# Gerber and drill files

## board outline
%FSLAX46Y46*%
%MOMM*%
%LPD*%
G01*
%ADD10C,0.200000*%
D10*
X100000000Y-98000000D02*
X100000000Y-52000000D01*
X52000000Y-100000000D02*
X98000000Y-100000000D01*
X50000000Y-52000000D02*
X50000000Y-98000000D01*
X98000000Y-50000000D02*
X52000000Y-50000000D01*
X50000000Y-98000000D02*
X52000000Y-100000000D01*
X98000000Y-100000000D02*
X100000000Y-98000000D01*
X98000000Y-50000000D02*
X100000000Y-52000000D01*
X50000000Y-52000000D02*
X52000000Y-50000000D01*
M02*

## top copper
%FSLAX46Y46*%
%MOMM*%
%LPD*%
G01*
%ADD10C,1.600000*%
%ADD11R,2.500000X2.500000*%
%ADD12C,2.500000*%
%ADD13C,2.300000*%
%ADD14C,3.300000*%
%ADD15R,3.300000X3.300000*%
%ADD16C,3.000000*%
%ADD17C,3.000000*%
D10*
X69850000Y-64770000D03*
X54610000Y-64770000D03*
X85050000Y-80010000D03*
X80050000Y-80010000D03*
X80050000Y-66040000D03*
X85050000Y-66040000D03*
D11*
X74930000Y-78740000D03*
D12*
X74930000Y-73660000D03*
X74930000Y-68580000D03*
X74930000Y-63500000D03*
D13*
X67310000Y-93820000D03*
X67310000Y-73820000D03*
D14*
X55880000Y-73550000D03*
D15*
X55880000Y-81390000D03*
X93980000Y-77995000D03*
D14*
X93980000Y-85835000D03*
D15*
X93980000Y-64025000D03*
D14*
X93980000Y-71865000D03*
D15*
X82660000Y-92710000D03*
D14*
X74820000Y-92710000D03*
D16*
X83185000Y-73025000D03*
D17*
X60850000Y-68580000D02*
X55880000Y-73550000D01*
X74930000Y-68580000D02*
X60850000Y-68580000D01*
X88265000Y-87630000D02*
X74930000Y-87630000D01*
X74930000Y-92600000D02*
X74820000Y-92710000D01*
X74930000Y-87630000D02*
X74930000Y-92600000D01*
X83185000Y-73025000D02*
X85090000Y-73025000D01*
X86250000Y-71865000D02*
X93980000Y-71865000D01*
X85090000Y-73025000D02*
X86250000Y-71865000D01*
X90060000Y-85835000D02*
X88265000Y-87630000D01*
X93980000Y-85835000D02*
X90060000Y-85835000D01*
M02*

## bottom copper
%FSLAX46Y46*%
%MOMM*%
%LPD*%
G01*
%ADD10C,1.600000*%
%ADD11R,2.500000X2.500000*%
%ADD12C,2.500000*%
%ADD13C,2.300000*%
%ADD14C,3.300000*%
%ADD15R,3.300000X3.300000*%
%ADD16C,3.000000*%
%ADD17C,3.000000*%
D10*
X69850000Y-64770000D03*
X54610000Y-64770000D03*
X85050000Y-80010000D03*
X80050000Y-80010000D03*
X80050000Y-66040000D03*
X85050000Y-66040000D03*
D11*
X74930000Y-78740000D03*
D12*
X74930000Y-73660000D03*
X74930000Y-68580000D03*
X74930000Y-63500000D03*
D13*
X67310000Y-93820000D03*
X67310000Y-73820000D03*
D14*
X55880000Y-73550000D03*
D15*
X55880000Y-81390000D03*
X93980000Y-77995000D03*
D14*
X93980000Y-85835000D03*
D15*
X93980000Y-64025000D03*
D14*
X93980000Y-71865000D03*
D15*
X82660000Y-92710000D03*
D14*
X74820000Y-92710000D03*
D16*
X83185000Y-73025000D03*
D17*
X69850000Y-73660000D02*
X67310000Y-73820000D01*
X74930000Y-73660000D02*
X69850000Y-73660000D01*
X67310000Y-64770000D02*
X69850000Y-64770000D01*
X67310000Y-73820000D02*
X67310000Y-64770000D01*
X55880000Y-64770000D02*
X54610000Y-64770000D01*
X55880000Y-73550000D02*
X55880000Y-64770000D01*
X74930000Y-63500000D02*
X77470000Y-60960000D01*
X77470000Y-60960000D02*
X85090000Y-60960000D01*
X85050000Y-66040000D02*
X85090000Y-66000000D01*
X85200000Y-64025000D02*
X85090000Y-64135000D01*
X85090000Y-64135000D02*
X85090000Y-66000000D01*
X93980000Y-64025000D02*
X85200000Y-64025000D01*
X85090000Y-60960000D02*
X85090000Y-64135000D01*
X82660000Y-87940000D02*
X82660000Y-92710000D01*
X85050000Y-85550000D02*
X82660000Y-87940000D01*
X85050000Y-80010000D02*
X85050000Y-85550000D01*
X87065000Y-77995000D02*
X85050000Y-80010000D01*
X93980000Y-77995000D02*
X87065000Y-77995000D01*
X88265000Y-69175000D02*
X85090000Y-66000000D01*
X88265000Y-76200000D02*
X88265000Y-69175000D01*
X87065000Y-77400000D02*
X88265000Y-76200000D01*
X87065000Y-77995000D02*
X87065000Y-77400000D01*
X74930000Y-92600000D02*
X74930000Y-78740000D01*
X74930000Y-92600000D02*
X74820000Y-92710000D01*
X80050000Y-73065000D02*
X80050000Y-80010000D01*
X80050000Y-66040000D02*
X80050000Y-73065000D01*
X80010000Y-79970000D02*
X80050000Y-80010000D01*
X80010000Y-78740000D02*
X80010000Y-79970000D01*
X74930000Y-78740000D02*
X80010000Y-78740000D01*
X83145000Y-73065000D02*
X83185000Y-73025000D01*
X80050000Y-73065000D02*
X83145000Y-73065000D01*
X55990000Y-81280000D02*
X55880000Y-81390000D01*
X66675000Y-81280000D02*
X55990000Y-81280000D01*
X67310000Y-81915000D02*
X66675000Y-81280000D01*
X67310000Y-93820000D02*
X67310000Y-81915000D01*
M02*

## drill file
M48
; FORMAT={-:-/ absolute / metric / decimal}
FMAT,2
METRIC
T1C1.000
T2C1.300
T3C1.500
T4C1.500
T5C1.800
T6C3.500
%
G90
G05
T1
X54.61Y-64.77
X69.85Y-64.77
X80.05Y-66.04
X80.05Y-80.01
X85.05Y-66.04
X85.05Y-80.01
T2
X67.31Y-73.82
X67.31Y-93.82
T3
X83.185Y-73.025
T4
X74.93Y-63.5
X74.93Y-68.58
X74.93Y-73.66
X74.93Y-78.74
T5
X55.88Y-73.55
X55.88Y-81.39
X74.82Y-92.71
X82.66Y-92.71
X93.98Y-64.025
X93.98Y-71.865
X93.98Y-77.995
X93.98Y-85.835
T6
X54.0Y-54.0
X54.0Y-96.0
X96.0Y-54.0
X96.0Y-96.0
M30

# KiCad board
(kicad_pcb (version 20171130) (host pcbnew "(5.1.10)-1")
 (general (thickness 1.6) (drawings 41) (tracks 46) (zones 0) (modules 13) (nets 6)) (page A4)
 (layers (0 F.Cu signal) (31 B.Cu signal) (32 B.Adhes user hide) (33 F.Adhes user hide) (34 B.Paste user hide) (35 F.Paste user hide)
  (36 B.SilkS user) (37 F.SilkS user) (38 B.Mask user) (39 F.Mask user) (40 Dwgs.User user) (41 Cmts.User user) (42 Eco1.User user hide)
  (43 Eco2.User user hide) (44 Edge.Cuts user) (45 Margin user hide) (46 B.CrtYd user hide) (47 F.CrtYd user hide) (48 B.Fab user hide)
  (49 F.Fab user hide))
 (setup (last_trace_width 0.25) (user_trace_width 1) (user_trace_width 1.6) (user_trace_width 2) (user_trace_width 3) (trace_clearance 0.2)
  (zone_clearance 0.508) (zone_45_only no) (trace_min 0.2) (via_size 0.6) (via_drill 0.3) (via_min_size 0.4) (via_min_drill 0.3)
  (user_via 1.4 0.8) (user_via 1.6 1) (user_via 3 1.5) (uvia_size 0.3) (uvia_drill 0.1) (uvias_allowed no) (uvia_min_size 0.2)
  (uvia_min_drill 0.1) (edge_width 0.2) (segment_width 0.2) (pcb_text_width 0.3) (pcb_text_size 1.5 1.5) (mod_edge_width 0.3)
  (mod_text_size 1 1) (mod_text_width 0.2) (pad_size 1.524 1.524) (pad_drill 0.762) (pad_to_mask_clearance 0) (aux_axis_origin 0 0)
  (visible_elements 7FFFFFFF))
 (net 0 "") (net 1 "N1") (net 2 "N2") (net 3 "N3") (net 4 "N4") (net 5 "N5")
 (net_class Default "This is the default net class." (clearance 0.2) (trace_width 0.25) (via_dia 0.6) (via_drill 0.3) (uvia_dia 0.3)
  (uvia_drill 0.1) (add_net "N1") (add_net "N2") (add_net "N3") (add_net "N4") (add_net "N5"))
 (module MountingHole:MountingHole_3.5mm (layer F.Cu) (at 54 96)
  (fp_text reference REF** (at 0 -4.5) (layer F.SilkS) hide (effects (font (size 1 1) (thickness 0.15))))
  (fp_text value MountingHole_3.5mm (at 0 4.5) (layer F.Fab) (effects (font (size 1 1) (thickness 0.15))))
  (pad 1 np_thru_hole circle (at 0 0) (size 3.5 3.5) (drill 3.5) (layers *.Cu *.Mask)))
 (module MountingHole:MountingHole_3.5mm (layer F.Cu) (at 96 96)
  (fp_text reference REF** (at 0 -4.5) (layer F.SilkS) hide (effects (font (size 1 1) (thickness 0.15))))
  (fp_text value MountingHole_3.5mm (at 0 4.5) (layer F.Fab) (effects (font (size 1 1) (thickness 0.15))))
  (pad 1 np_thru_hole circle (at 0 0) (size 3.5 3.5) (drill 3.5) (layers *.Cu *.Mask)))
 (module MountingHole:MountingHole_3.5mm (layer F.Cu) (at 96 54)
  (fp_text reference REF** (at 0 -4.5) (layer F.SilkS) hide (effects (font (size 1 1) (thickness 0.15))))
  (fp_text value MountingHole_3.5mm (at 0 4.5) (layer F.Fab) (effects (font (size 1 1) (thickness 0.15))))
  (pad 1 np_thru_hole circle (at 0 0) (size 3.5 3.5) (drill 3.5) (layers *.Cu *.Mask)))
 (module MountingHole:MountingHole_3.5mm (layer F.Cu) (at 54 54)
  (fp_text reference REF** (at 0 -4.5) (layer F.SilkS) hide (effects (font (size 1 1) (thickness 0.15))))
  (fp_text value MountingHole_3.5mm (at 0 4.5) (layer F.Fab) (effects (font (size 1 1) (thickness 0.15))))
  (pad 1 np_thru_hole circle (at 0 0) (size 3.5 3.5) (drill 3.5) (layers *.Cu *.Mask)))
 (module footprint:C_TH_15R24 (layer F.Cu) (at 62.23 64.77 180)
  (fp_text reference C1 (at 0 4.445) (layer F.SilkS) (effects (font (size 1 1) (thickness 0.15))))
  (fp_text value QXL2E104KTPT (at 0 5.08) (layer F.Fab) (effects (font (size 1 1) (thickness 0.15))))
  (pad 1 thru_hole circle (at -7.62 0 180) (size 1.6 1.6) (drill 1) (layers *.Cu *.Mask) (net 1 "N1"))
  (pad 2 thru_hole circle (at 7.62 0 180) (size 1.6 1.6) (drill 1) (layers *.Cu *.Mask) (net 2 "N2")))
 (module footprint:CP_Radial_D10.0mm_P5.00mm (layer F.Cu) (at 82.55 80.01 180)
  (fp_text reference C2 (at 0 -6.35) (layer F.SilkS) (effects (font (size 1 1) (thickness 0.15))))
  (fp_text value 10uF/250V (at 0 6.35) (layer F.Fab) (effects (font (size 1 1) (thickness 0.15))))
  (pad 1 thru_hole circle (at -2.5 0 180) (size 1.6 1.6) (drill 1) (layers *.Cu *.Mask) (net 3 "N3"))
  (pad 2 thru_hole circle (at 2.5 0 180) (size 1.6 1.6) (drill 1) (layers *.Cu *.Mask) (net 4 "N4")))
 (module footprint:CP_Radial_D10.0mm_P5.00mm (layer F.Cu) (at 82.55 66.04 180)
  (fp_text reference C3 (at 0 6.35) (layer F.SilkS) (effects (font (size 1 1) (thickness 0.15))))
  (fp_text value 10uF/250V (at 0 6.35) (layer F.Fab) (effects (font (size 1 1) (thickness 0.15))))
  (pad 2 thru_hole circle (at 2.5 0 180) (size 1.6 1.6) (drill 1) (layers *.Cu *.Mask) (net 4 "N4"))
  (pad 1 thru_hole circle (at -2.5 0 180) (size 1.6 1.6) (drill 1) (layers *.Cu *.Mask) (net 3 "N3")))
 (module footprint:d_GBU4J (layer F.Cu) (at 74.93 71.12 90)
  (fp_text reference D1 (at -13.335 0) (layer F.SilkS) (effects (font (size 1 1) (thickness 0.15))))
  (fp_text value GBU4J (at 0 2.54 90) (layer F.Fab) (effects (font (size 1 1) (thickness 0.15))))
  (pad 1 thru_hole rect (at -7.62 0 90) (size 2.5 2.5) (drill 1.5) (layers *.Cu *.Mask) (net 4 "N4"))
  (pad 2 thru_hole circle (at -2.54 0 90) (size 2.5 2.5) (drill 1.5) (layers *.Cu *.Mask) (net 1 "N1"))
  (pad 3 thru_hole circle (at 2.54 0 90) (size 2.5 2.5) (drill 1.5) (layers *.Cu *.Mask) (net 2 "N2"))
  (pad 4 thru_hole circle (at 7.62 0 90) (size 2.5 2.5) (drill 1.5) (layers *.Cu *.Mask) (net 3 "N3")))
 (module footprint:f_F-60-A (layer F.Cu) (at 67.31 83.82 90)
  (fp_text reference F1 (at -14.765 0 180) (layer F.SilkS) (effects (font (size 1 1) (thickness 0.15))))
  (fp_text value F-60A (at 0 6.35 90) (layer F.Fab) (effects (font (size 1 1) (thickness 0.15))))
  (pad 1 thru_hole circle (at -10 0 90) (size 2.3 2.3) (drill 1.3) (layers *.Cu *.Mask) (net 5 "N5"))
  (pad 2 thru_hole circle (at 10 0 90) (size 2.3 2.3) (drill 1.3) (layers *.Cu *.Mask) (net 1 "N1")))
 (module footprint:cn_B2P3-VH (layer F.Cu) (at 55.88 77.47 90)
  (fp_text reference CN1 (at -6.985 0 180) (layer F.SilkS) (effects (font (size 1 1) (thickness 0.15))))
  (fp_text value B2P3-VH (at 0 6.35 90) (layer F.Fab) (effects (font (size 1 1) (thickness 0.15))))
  (pad 2 thru_hole circle (at 3.92 0 90) (size 3.3 3.3) (drill 1.8) (layers *.Cu *.Mask) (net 2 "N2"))
  (pad 1 thru_hole rect (at -3.92 0 90) (size 3.3 3.3) (drill 1.8) (layers *.Cu *.Mask) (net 5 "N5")))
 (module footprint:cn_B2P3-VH (layer F.Cu) (at 93.98 81.915 270)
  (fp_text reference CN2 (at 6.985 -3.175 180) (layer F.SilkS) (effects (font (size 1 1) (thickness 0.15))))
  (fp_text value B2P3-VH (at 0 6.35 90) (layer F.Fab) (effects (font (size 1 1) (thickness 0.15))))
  (pad 1 thru_hole rect (at -3.92 0 270) (size 3.3 3.3) (drill 1.8) (layers *.Cu *.Mask) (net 3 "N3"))
  (pad 2 thru_hole circle (at 3.92 0 270) (size 3.3 3.3) (drill 1.8) (layers *.Cu *.Mask) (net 4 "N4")))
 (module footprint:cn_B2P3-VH (layer F.Cu) (at 93.98 67.945 270)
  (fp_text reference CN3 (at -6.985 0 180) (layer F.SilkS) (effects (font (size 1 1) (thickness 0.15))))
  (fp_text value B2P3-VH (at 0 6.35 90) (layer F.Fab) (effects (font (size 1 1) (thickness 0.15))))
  (pad 1 thru_hole rect (at -3.92 0 270) (size 3.3 3.3) (drill 1.8) (layers *.Cu *.Mask) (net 3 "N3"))
  (pad 2 thru_hole circle (at 3.92 0 270) (size 3.3 3.3) (drill 1.8) (layers *.Cu *.Mask) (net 4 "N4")))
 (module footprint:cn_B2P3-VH (layer F.Cu) (at 78.74 92.71 180)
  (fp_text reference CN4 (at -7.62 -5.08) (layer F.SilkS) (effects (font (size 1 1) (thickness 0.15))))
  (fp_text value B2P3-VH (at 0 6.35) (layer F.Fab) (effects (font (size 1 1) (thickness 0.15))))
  (pad 1 thru_hole rect (at -3.92 0 180) (size 3.3 3.3) (drill 1.8) (layers *.Cu *.Mask) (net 3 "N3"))
  (pad 2 thru_hole circle (at 3.92 0 180) (size 3.3 3.3) (drill 1.8) (layers *.Cu *.Mask) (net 4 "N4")))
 (gr_line (start 100 98) (end 100 52) (layer Edge.Cuts) (width 0.2))
 (gr_line (start 52 100) (end 98 100) (layer Edge.Cuts) (width 0.2))
 (gr_line (start 50 52) (end 50 98) (layer Edge.Cuts) (width 0.2))
 (gr_line (start 98 50) (end 52 50) (layer Edge.Cuts) (width 0.2))
 (gr_line (start 50 98) (end 52 100) (layer Edge.Cuts) (width 0.2))
 (gr_line (start 98 100) (end 100 98) (layer Edge.Cuts) (width 0.2))
 (gr_line (start 98 50) (end 100 52) (layer Edge.Cuts) (width 0.2))
 (gr_line (start 50 52) (end 52 50) (layer Edge.Cuts) (width 0.2))
 (segment (start 69.85 73.66) (end 67.31 73.82) (width 3) (layer B.Cu) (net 1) (status 20))
 (segment (start 74.93 73.66) (end 69.85 73.66) (width 3) (layer B.Cu) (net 1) (status 10))
 (segment (start 67.31 64.77) (end 69.85 64.77) (width 3) (layer B.Cu) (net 1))
 (segment (start 67.31 73.82) (end 67.31 64.77) (width 3) (layer B.Cu) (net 1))
 (segment (start 55.88 64.77) (end 54.61 64.77) (width 3) (layer B.Cu) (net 2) (status 20))
 (segment (start 55.88 73.55) (end 55.88 64.77) (width 3) (layer B.Cu) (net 2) (status 10))
 (segment (start 60.85 68.58) (end 55.88 73.55) (width 3) (layer F.Cu) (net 2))
 (segment (start 74.93 68.58) (end 60.85 68.58) (width 3) (layer F.Cu) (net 2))
 (segment (start 74.93 63.5) (end 77.47 60.96) (width 3) (layer B.Cu) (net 3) (status 10))
 (segment (start 77.47 60.96) (end 85.09 60.96) (width 3) (layer B.Cu) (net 3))
 (segment (start 85.05 66.04) (end 85.09 66) (width 3) (layer B.Cu) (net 3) (status 30))
 (segment (start 85.2 64.025) (end 85.09 64.135) (width 3) (layer B.Cu) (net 3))
 (segment (start 85.09 64.135) (end 85.09 66) (width 3) (layer B.Cu) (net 3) (status 20))
 (segment (start 93.98 64.025) (end 85.2 64.025) (width 3) (layer B.Cu) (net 3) (status 10))
 (segment (start 85.09 60.96) (end 85.09 64.135) (width 3) (layer B.Cu) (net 3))
 (segment (start 82.66 87.94) (end 82.66 92.71) (width 3) (layer B.Cu) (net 3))
 (segment (start 85.05 85.55) (end 82.66 87.94) (width 3) (layer B.Cu) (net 3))
 (segment (start 85.05 80.01) (end 85.05 85.55) (width 3) (layer B.Cu) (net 3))
 (segment (start 87.065 77.995) (end 85.05 80.01) (width 3) (layer B.Cu) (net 3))
 (segment (start 93.98 77.995) (end 87.065 77.995) (width 3) (layer B.Cu) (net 3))
 (segment (start 88.265 69.175) (end 85.09 66) (width 3) (layer B.Cu) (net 3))
 (segment (start 88.265 76.2) (end 88.265 69.175) (width 3) (layer B.Cu) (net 3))
 (segment (start 87.065 77.4) (end 88.265 76.2) (width 3) (layer B.Cu) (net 3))
 (segment (start 87.065 77.995) (end 87.065 77.4) (width 3) (layer B.Cu) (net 3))
 (segment (start 74.93 92.6) (end 74.93 78.74) (width 3) (layer B.Cu) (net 4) (status 30))
 (segment (start 74.93 92.6) (end 74.82 92.71) (width 3) (layer B.Cu) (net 4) (status 30))
 (segment (start 88.265 87.63) (end 74.93 87.63) (width 3) (layer F.Cu) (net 4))
 (segment (start 74.93 92.6) (end 74.82 92.71) (width 3) (layer F.Cu) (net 4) (status 30))
 (segment (start 74.93 87.63) (end 74.93 92.6) (width 3) (layer F.Cu) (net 4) (status 20))
 (segment (start 80.05 73.065) (end 80.05 80.01) (width 3) (layer B.Cu) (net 4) (status 20))
 (segment (start 80.05 66.04) (end 80.05 73.065) (width 3) (layer B.Cu) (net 4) (status 10))
 (segment (start 80.01 79.97) (end 80.05 80.01) (width 3) (layer B.Cu) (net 4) (status 30))
 (segment (start 80.01 78.74) (end 80.01 79.97) (width 3) (layer B.Cu) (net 4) (status 20))
 (segment (start 74.93 78.74) (end 80.01 78.74) (width 3) (layer B.Cu) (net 4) (status 10))
 (via (at 83.185 73.025) (size 3) (drill 1.5) (layers F.Cu B.Cu) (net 4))
 (segment (start 83.145 73.065) (end 83.185 73.025) (width 3) (layer B.Cu) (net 4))
 (segment (start 80.05 73.065) (end 83.145 73.065) (width 3) (layer B.Cu) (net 4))
 (segment (start 83.185 73.025) (end 85.09 73.025) (width 3) (layer F.Cu) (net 4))
 (segment (start 86.25 71.865) (end 93.98 71.865) (width 3) (layer F.Cu) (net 4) (status 20))
 (segment (start 85.09 73.025) (end 86.25 71.865) (width 3) (layer F.Cu) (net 4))
 (segment (start 90.06 85.835) (end 88.265 87.63) (width 3) (layer F.Cu) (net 4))
 (segment (start 93.98 85.835) (end 90.06 85.835) (width 3) (layer F.Cu) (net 4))
 (segment (start 55.99 81.28) (end 55.88 81.39) (width 3) (layer B.Cu) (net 5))
 (segment (start 66.675 81.28) (end 55.99 81.28) (width 3) (layer B.Cu) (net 5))
 (segment (start 67.31 81.915) (end 66.675 81.28) (width 3) (layer B.Cu) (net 5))
 (segment (start 67.31 93.82) (end 67.31 81.915) (width 3) (layer B.Cu) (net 5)))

